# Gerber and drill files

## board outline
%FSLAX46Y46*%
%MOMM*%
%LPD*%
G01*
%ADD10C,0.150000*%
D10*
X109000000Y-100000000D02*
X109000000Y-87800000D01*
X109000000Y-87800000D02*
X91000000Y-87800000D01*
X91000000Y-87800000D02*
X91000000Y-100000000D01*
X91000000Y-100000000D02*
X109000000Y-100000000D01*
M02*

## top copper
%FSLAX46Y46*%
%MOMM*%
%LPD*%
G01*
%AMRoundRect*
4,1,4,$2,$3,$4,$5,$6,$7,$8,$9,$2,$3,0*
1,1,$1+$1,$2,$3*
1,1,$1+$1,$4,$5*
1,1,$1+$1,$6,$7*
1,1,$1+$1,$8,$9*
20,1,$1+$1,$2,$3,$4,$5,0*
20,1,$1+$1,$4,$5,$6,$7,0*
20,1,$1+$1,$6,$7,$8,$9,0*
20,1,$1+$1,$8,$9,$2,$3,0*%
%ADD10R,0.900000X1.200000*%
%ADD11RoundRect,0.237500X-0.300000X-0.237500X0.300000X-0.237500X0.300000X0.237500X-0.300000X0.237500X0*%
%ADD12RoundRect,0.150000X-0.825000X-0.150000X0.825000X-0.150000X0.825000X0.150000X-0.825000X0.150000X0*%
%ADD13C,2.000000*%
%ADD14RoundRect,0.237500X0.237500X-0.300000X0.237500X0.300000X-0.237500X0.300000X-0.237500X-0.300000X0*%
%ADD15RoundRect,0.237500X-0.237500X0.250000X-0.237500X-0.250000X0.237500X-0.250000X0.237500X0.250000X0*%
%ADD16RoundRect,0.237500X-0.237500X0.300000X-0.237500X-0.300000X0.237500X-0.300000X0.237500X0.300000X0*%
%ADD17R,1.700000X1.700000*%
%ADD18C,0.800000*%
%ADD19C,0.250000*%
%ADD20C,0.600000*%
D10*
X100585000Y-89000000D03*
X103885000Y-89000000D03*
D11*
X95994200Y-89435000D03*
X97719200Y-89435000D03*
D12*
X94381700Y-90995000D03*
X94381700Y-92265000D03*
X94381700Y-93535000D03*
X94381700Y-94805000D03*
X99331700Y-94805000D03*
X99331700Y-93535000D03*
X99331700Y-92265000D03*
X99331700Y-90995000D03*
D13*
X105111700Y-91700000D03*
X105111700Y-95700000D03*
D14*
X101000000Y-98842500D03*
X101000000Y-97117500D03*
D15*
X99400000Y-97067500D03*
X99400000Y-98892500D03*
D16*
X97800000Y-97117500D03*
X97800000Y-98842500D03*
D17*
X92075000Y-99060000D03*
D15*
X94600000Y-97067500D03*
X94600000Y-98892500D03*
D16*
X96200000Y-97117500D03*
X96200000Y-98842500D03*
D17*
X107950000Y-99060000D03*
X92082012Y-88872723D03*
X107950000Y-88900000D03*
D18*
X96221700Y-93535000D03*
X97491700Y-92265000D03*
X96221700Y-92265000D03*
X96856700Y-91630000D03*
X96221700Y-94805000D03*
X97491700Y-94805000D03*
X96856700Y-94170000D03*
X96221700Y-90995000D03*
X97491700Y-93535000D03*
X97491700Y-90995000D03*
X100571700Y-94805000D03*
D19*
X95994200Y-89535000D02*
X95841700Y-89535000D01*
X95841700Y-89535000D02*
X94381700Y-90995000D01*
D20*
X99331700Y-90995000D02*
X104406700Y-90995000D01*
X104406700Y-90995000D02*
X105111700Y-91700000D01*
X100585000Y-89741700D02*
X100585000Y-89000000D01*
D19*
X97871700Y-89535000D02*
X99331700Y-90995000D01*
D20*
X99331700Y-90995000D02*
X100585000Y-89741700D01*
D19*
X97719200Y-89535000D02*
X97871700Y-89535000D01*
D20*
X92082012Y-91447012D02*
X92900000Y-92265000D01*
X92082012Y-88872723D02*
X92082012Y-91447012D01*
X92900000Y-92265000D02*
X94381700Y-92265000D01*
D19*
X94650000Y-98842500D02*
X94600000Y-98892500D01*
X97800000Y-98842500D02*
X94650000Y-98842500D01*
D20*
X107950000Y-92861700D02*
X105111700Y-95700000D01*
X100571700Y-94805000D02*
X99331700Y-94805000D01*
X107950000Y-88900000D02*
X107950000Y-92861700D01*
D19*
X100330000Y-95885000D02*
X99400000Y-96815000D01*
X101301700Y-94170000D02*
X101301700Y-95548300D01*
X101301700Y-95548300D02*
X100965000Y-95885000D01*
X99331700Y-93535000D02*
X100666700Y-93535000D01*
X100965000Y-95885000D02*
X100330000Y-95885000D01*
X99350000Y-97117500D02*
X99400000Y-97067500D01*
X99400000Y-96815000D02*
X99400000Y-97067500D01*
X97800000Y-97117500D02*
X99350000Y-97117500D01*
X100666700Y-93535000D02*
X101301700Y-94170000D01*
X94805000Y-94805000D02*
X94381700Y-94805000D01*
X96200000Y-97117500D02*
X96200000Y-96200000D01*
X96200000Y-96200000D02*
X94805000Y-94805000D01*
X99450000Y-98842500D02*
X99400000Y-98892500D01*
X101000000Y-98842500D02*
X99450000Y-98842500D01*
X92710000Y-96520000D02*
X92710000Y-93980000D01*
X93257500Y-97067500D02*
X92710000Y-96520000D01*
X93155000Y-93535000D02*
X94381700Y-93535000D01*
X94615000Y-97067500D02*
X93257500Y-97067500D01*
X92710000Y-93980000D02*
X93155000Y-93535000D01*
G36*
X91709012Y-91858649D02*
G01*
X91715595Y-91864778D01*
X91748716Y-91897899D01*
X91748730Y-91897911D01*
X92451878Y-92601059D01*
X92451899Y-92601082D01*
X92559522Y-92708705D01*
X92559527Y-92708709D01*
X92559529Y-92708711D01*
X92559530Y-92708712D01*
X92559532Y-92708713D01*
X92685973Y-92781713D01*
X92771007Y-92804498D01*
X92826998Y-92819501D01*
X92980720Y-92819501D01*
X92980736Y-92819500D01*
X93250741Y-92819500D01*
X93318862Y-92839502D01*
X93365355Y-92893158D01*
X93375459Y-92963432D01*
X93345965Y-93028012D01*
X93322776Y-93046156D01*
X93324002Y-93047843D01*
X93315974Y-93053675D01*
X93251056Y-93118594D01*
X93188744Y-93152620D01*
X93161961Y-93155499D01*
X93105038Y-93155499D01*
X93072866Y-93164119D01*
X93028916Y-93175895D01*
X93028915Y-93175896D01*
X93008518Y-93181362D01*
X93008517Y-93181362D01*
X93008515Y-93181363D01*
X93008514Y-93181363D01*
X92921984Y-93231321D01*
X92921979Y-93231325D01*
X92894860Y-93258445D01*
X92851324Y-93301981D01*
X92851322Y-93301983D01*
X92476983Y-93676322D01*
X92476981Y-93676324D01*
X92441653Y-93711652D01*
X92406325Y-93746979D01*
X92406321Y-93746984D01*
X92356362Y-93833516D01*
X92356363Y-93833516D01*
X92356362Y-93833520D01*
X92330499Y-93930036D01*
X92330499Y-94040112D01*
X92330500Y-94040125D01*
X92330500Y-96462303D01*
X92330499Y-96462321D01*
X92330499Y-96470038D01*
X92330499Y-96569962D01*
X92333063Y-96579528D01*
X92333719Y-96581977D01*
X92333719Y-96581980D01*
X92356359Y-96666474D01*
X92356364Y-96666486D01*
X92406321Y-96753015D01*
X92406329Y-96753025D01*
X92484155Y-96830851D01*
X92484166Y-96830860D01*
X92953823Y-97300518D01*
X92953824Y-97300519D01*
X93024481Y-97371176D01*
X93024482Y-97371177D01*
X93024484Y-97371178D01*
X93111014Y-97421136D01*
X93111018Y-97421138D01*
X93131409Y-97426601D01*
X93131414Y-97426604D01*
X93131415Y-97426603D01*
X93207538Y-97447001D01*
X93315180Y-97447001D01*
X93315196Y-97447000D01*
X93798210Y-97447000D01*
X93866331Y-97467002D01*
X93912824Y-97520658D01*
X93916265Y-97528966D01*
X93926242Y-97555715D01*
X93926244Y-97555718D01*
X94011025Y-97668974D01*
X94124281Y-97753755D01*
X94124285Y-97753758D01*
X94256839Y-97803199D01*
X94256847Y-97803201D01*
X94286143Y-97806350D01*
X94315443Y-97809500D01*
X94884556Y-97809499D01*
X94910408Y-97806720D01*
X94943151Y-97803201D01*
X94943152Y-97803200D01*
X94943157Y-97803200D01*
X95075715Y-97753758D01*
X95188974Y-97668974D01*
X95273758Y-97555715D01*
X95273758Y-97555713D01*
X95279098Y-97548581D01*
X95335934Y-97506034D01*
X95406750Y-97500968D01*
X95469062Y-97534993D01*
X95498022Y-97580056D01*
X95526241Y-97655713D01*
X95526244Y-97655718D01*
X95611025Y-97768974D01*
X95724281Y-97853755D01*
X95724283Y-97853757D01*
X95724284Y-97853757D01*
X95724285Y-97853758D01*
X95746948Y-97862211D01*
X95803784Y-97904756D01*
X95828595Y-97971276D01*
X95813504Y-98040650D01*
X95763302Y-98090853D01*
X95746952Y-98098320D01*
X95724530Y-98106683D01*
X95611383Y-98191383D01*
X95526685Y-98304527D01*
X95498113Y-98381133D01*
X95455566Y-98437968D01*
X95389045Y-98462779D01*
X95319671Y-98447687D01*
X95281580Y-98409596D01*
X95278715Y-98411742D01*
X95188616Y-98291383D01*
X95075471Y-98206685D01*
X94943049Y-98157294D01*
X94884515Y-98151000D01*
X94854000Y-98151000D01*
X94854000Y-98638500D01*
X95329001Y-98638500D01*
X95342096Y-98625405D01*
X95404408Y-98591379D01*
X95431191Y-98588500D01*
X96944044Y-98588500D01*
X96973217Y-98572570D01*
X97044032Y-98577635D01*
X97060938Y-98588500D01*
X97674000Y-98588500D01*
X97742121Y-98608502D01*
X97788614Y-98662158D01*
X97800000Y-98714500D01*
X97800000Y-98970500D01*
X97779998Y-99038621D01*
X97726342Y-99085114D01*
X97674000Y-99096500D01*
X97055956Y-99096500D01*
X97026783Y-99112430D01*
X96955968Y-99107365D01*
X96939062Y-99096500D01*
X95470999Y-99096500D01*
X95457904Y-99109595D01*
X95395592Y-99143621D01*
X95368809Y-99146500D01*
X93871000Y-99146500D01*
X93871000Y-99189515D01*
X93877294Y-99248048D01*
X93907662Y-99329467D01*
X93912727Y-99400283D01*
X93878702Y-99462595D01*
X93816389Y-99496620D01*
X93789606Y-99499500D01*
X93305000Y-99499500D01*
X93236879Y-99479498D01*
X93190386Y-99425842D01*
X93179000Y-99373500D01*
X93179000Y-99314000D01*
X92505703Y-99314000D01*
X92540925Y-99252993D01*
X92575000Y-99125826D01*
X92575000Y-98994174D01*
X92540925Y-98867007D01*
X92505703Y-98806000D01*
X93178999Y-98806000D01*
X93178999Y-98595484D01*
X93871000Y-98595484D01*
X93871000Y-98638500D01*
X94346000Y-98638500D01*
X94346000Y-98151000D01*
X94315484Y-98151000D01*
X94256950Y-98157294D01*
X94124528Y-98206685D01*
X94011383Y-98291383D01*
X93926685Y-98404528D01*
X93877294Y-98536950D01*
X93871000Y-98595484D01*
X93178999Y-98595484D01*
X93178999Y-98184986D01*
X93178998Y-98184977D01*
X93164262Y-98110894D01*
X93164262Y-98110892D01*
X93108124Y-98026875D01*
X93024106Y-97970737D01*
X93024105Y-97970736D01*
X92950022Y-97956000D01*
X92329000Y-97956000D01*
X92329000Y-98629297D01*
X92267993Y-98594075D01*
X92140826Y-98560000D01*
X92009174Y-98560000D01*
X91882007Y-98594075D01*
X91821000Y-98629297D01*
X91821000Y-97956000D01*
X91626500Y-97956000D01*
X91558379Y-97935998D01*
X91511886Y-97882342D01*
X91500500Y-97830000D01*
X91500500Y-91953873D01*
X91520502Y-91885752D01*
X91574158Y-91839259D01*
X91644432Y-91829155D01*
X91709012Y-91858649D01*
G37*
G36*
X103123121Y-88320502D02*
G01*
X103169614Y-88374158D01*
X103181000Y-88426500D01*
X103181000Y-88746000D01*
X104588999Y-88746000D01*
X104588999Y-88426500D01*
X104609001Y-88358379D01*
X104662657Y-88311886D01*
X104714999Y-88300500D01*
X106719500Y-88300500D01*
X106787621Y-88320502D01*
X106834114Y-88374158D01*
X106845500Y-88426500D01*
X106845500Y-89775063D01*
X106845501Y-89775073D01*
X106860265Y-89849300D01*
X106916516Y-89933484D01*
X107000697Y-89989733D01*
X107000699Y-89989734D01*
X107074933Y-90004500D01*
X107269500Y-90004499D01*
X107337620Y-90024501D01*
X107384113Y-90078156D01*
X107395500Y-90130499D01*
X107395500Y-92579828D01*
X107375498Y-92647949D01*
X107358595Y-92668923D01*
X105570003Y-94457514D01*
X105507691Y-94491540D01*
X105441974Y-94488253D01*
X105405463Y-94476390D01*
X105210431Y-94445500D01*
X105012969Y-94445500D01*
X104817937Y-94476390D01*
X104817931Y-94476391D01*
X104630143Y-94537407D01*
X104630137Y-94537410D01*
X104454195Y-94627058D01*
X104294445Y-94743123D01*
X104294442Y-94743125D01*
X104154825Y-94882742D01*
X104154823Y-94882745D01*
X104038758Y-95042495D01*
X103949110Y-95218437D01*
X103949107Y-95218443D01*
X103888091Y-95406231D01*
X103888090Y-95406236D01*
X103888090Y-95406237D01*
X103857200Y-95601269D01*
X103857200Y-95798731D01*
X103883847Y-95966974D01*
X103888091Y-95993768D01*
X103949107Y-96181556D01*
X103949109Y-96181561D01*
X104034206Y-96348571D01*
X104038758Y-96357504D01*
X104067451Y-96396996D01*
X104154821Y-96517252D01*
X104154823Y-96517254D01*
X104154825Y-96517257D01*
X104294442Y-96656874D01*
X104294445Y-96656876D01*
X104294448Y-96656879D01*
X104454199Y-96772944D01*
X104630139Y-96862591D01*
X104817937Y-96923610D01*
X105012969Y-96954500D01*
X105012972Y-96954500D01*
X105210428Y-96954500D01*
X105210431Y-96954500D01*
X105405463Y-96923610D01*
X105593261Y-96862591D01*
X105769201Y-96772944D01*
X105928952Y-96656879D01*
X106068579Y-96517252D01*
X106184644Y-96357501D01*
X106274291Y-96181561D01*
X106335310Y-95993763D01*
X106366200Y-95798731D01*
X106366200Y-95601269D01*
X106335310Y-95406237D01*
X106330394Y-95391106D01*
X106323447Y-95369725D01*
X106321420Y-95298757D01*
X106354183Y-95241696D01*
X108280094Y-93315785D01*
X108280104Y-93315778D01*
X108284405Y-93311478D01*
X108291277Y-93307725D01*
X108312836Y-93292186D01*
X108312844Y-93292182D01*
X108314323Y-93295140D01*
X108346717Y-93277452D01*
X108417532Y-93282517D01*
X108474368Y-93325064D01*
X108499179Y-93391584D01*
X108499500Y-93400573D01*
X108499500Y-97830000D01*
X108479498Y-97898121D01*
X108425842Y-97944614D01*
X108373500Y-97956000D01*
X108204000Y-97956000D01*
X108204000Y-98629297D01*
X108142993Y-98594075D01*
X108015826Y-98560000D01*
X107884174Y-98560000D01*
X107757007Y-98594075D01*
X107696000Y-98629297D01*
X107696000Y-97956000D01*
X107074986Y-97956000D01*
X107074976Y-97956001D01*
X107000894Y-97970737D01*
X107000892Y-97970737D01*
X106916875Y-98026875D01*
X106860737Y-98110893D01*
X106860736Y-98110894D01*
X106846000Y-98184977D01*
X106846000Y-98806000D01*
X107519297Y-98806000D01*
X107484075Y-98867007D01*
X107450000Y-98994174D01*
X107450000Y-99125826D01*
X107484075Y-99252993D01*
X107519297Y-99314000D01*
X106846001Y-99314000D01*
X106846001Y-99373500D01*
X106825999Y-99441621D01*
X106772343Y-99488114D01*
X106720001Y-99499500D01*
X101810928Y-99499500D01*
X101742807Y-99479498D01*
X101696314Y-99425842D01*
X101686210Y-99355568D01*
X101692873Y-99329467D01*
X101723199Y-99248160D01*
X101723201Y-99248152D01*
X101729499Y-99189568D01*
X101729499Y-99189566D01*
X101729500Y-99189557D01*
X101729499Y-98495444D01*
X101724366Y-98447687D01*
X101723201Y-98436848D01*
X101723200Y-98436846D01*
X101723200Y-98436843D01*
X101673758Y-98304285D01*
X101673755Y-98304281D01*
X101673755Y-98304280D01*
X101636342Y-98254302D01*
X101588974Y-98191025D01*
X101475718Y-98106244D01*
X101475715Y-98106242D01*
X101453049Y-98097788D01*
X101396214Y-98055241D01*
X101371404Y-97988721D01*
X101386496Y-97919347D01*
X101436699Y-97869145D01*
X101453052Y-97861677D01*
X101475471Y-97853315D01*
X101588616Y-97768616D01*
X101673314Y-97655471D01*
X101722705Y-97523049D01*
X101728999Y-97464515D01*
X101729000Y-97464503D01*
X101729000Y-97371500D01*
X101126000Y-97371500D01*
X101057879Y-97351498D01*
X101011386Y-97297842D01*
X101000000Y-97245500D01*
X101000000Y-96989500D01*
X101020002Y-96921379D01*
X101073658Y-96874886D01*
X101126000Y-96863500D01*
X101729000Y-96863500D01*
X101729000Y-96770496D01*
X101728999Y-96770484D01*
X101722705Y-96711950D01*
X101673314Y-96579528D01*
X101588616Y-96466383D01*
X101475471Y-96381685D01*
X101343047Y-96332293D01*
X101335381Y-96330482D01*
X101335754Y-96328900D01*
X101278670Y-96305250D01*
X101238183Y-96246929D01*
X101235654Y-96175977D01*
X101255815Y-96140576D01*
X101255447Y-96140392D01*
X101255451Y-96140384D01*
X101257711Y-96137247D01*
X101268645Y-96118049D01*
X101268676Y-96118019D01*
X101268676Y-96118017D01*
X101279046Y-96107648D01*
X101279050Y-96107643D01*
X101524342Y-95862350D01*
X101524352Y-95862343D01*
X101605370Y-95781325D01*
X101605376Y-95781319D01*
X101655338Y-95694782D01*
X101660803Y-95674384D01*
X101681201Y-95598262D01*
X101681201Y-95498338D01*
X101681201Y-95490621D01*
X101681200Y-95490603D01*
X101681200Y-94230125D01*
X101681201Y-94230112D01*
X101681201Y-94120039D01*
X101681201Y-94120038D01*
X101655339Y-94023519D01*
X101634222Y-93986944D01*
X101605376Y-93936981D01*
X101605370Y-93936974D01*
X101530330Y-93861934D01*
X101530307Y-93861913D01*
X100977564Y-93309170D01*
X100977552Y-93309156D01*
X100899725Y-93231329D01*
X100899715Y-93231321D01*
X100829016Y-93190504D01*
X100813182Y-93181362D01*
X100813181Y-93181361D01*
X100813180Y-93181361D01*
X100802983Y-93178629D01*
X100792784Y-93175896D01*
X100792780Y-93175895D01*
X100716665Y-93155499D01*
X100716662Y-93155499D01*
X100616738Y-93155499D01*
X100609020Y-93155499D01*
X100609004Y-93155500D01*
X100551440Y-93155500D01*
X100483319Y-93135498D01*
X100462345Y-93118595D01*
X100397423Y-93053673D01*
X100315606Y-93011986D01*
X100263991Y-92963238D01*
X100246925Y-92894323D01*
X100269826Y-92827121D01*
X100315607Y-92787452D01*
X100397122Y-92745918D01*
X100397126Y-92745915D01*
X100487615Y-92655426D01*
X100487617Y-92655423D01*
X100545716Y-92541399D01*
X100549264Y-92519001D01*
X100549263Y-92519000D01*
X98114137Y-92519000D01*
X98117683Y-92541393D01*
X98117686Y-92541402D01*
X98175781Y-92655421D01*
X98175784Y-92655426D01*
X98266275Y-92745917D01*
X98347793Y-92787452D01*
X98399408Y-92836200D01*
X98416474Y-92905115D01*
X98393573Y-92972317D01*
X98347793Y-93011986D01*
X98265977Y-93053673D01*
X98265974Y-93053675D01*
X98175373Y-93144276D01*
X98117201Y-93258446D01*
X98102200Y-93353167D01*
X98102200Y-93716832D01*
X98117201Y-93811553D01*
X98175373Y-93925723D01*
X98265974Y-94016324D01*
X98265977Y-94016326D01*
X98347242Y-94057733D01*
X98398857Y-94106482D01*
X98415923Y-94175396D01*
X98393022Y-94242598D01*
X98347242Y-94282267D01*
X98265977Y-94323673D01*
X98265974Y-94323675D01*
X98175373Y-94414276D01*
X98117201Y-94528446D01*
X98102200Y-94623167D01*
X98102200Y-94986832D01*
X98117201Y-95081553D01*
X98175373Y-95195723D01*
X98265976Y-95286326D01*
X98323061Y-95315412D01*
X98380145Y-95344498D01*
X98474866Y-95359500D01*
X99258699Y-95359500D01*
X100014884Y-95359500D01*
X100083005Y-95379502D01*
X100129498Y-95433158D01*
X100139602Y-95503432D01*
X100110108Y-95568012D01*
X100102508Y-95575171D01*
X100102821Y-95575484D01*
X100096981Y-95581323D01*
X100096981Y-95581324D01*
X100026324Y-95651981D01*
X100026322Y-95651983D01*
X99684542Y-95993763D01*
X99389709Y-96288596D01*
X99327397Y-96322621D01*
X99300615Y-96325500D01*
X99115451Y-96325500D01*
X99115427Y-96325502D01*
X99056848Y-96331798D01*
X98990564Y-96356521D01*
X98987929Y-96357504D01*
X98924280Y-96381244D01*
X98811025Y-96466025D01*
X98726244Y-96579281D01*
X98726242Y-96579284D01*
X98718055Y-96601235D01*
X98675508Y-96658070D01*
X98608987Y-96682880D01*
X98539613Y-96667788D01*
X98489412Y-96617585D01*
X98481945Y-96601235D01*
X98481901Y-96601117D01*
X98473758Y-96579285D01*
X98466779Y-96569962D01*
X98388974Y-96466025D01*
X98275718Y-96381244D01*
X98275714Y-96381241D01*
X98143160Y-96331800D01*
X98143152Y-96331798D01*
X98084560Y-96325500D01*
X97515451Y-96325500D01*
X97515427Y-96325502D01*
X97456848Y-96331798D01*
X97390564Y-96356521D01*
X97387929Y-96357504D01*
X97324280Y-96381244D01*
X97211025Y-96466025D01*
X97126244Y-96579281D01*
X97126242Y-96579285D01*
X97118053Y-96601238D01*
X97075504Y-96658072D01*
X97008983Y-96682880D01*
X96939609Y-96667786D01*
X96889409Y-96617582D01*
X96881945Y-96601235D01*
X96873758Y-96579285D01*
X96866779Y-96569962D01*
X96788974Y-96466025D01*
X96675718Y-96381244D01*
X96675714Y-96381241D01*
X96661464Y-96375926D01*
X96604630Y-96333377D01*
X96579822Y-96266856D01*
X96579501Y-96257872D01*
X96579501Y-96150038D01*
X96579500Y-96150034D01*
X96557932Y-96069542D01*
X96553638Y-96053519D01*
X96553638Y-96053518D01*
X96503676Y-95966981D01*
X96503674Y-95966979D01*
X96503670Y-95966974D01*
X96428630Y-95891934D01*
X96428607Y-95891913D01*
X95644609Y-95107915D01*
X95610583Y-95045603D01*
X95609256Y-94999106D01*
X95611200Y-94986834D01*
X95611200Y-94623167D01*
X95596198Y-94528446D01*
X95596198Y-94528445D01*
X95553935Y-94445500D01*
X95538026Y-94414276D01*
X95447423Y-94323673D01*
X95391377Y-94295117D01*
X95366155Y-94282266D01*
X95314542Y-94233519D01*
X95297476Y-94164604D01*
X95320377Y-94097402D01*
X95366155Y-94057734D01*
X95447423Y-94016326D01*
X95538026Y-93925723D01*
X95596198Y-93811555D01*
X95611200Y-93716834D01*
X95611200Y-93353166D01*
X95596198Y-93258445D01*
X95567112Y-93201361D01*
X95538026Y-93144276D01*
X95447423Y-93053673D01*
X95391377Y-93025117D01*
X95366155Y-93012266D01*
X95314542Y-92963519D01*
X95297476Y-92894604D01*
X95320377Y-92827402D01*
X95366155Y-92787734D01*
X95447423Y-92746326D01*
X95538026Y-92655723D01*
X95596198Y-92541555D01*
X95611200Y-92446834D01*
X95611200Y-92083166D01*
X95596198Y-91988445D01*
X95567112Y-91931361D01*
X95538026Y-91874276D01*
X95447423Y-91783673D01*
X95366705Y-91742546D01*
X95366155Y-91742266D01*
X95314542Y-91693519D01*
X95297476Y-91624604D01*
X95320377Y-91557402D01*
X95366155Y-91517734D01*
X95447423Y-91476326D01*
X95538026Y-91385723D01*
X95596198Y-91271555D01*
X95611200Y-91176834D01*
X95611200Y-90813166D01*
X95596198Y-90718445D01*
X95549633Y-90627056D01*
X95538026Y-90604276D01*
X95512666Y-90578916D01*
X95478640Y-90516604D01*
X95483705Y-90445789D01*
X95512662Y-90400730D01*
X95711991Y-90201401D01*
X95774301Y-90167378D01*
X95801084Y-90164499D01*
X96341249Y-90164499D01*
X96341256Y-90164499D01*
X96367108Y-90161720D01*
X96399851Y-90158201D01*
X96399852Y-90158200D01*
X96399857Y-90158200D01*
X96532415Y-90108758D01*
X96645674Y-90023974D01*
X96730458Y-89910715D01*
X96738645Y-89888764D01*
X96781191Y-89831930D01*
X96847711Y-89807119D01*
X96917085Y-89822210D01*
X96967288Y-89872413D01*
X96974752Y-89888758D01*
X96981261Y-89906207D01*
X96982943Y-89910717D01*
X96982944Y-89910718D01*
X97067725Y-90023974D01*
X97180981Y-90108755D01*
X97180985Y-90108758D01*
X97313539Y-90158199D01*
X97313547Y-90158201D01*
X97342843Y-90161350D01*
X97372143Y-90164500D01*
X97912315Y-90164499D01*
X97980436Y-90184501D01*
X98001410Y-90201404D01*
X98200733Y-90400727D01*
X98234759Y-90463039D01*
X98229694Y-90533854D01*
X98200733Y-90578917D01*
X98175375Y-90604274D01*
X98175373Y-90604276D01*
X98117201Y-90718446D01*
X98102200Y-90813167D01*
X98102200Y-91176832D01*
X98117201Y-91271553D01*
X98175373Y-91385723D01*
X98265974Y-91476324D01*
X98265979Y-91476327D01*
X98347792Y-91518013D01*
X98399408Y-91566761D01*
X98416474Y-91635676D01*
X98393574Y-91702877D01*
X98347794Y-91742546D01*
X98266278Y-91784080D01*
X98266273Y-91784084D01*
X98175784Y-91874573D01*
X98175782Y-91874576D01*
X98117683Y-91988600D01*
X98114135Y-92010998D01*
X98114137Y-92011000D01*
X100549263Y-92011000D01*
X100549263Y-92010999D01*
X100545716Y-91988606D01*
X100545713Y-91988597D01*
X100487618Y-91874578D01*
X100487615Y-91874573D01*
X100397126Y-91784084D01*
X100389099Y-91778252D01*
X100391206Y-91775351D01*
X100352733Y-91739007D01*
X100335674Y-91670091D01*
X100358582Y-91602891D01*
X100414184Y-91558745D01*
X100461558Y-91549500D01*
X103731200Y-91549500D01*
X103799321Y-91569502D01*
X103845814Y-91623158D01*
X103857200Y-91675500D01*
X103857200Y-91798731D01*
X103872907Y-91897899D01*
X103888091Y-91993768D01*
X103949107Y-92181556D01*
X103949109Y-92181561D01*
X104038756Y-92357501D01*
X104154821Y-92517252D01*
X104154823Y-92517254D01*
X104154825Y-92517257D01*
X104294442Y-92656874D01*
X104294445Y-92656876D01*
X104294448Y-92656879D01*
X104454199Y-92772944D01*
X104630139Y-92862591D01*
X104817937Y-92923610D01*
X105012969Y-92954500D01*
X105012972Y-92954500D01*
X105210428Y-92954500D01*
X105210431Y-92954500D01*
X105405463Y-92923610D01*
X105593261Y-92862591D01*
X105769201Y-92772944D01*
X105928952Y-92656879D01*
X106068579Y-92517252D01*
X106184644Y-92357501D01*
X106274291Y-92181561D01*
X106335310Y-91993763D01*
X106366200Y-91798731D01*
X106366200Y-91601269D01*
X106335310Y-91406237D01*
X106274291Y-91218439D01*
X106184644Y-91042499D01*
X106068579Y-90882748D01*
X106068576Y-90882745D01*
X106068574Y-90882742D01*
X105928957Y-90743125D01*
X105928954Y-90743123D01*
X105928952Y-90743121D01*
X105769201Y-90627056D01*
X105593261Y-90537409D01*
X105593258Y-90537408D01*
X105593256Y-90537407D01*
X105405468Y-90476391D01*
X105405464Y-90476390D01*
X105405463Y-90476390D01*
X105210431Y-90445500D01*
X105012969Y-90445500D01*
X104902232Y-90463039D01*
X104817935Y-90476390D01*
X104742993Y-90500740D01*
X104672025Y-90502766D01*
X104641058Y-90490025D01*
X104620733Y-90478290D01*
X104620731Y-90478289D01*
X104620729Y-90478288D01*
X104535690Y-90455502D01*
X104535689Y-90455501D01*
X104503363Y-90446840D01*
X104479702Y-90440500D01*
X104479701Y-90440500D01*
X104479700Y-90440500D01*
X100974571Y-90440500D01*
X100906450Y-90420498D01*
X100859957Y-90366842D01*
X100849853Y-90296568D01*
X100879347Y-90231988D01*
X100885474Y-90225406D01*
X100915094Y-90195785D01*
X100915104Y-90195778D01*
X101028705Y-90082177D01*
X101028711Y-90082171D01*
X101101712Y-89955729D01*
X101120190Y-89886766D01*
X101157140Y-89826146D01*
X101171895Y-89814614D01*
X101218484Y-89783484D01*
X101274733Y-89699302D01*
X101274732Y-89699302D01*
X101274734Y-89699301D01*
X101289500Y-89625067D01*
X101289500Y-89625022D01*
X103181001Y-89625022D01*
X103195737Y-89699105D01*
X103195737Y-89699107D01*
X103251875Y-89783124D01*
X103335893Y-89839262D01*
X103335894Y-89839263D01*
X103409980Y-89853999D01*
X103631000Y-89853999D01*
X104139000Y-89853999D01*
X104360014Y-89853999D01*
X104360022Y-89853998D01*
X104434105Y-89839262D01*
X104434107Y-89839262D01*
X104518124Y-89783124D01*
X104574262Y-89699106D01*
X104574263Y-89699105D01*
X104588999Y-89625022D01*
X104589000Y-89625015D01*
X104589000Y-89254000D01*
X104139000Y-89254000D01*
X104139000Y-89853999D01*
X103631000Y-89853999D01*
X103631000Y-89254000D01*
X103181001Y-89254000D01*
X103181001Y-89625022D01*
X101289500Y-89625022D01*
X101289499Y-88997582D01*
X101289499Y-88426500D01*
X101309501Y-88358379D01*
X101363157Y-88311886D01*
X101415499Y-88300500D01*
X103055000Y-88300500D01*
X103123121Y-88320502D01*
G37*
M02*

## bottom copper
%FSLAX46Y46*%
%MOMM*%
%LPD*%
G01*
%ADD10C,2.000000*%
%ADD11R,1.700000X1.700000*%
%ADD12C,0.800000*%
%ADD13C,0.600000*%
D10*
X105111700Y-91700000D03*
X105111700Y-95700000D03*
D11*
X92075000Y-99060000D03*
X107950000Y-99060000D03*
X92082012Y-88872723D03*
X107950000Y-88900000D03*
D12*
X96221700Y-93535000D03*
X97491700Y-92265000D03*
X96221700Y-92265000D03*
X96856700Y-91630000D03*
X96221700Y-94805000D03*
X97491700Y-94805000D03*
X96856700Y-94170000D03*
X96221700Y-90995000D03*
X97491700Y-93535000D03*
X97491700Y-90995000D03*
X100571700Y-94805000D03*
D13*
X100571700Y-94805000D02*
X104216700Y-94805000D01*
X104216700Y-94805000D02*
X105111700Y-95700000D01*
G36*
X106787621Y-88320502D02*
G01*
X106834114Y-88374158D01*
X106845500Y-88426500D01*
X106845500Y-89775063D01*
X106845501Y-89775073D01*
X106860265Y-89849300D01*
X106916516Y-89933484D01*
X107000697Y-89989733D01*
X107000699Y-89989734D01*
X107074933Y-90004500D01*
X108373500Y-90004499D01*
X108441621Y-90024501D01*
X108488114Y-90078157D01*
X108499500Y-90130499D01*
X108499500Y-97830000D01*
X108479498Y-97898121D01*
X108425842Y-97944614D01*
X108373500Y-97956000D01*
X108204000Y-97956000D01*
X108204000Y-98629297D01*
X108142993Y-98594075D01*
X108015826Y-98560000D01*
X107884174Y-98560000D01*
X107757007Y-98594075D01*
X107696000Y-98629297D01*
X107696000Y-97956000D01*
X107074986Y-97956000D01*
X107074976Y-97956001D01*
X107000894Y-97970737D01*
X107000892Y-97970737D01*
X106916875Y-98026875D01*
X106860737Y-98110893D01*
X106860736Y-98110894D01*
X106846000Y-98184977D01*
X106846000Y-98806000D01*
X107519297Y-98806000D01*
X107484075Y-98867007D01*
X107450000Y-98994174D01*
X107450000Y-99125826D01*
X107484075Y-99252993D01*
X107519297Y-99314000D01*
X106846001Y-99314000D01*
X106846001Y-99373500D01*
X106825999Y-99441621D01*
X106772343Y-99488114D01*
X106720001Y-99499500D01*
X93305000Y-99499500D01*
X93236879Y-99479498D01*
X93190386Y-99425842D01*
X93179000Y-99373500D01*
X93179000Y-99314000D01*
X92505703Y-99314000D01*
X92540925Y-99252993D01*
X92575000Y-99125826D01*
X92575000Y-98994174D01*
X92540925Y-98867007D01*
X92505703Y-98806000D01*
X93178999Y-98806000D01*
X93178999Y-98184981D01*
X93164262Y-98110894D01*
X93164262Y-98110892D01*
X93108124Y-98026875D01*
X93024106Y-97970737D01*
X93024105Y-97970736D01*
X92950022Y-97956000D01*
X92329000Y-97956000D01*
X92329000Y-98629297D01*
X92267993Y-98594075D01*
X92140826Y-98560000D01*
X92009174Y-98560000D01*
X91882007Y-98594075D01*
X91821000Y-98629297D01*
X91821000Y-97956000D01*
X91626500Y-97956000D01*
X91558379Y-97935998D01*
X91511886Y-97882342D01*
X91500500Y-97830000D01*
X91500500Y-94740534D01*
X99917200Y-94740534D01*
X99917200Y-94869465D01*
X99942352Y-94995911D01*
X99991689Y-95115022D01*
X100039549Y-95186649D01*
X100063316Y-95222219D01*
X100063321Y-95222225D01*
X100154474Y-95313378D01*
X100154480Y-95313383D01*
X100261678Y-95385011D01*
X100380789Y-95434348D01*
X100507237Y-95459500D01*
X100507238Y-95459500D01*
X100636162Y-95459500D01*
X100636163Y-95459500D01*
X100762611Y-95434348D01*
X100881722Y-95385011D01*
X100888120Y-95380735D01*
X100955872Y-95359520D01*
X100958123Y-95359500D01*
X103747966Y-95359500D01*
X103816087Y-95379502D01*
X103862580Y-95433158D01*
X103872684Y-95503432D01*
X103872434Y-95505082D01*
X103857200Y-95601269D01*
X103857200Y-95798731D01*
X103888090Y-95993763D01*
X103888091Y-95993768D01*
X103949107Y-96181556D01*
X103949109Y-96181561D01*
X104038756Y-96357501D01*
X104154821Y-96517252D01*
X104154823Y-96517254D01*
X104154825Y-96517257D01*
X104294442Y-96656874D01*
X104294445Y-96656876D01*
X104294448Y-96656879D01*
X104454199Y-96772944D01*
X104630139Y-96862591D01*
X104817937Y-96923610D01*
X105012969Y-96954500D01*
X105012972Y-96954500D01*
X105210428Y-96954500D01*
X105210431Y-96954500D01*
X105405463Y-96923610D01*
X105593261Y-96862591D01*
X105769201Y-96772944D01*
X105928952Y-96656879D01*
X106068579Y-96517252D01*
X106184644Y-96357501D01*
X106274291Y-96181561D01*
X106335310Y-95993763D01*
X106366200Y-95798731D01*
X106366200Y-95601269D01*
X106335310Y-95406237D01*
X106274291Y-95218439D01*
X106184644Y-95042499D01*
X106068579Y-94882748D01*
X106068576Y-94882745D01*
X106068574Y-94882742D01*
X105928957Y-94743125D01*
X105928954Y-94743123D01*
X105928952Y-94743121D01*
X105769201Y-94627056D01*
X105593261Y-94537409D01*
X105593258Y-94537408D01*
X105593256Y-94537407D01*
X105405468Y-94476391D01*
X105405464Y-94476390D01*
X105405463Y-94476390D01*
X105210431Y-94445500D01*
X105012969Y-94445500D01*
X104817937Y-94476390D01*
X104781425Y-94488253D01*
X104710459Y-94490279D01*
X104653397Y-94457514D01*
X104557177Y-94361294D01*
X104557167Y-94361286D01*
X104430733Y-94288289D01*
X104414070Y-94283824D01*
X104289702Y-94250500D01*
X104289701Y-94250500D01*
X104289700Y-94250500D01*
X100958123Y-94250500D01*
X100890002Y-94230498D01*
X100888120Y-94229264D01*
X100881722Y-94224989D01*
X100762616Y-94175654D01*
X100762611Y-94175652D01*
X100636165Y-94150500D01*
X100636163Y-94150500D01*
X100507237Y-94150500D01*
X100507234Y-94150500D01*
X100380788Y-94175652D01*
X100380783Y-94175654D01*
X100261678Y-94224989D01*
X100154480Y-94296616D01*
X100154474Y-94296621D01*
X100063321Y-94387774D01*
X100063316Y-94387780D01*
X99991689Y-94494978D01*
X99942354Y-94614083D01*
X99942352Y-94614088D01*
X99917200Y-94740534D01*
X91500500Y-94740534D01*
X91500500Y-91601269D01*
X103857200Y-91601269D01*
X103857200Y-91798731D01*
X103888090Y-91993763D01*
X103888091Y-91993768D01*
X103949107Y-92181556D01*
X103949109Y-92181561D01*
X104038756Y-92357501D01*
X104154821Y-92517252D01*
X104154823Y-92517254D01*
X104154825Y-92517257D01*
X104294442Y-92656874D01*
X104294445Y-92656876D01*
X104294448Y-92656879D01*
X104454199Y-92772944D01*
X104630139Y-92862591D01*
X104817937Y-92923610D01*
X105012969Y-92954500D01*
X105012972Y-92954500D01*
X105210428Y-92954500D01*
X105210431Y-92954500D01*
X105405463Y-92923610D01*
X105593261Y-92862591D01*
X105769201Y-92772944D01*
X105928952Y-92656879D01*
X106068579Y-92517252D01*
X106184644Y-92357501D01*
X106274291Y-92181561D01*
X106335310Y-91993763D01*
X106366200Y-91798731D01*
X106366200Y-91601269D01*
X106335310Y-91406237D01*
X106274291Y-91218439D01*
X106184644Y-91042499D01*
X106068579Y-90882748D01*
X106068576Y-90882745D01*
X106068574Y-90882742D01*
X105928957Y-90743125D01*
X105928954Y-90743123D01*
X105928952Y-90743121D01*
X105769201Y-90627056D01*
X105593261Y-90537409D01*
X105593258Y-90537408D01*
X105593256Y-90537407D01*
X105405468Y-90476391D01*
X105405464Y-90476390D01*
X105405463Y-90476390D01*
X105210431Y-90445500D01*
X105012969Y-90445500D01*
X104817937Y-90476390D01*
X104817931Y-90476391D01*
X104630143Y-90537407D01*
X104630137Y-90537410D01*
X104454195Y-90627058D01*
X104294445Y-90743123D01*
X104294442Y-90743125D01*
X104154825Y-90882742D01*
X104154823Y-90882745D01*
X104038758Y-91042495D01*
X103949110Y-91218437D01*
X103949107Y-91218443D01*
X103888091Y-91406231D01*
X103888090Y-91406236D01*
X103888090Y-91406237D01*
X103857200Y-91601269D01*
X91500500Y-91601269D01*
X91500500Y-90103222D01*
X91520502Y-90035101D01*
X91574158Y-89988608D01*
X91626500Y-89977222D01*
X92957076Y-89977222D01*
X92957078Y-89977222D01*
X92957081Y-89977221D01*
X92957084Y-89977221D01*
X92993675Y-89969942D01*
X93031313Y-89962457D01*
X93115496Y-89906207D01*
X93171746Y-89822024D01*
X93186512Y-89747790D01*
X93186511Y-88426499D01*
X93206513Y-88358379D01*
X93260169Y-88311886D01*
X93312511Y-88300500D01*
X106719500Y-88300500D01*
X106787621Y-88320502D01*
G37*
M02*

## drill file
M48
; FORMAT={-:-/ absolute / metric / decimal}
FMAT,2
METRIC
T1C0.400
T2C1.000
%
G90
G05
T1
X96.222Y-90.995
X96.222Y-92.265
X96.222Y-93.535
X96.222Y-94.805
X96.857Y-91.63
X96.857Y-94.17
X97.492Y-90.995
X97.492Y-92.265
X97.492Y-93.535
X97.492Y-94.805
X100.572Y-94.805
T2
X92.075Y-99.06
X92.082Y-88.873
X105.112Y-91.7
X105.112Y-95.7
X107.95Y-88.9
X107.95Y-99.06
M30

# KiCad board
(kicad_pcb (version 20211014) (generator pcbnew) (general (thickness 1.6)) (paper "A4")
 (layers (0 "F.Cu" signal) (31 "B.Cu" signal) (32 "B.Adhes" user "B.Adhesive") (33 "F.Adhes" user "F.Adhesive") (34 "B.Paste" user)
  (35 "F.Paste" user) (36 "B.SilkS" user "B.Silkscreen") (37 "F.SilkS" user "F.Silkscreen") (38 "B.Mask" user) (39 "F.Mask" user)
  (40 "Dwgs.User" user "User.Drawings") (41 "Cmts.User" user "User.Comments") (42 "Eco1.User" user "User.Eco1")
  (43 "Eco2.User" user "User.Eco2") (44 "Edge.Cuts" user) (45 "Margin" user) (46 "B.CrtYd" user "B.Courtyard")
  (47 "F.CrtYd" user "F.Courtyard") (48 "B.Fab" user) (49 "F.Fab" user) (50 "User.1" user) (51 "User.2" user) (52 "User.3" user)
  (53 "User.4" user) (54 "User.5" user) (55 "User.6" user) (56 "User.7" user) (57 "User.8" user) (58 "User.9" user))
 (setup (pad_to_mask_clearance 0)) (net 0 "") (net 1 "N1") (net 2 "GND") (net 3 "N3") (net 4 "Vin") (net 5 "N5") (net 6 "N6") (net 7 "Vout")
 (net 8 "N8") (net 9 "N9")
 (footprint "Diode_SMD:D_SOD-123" (layer "F.Cu") (at 102.235 89)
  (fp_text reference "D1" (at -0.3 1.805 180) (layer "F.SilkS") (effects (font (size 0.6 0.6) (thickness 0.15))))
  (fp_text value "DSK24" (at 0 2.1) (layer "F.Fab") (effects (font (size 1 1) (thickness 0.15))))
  (pad "1" smd rect (at -1.65 0) (size 0.9 1.2) (layers "F.Cu" "F.Paste" "F.Mask") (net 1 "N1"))
  (pad "2" smd rect (at 1.65 0) (size 0.9 1.2) (layers "F.Cu" "F.Paste" "F.Mask") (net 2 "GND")))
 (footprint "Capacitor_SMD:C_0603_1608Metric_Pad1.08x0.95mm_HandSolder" (layer "F.Cu") (at 96.8567 89.435)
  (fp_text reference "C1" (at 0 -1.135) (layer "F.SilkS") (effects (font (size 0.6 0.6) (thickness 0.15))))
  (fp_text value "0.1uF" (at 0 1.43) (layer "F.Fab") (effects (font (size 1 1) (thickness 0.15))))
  (pad "1" smd roundrect (at -0.8625 0) (size 1.075 0.95) (layers "F.Cu" "F.Paste" "F.Mask") (roundrect_rratio 0.25) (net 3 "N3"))
  (pad "2" smd roundrect (at 0.8625 0) (size 1.075 0.95) (layers "F.Cu" "F.Paste" "F.Mask") (roundrect_rratio 0.25) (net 1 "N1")))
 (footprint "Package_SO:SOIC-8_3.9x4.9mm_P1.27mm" (layer "F.Cu") (at 96.8567 92.9)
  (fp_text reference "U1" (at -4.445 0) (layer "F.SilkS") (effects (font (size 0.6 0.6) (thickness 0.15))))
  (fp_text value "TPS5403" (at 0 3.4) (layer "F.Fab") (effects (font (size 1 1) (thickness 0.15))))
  (pad "1" smd roundrect (at -2.475 -1.905) (size 1.95 0.6) (layers "F.Cu" "F.Paste" "F.Mask") (roundrect_rratio 0.25) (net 3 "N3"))
  (pad "2" smd roundrect (at -2.475 -0.635) (size 1.95 0.6) (layers "F.Cu" "F.Paste" "F.Mask") (roundrect_rratio 0.25) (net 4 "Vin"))
  (pad "3" smd roundrect (at -2.475 0.635) (size 1.95 0.6) (layers "F.Cu" "F.Paste" "F.Mask") (roundrect_rratio 0.25) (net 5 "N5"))
  (pad "4" smd roundrect (at -2.475 1.905) (size 1.95 0.6) (layers "F.Cu" "F.Paste" "F.Mask") (roundrect_rratio 0.25) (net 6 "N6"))
  (pad "5" smd roundrect (at 2.475 1.905) (size 1.95 0.6) (layers "F.Cu" "F.Paste" "F.Mask") (roundrect_rratio 0.25) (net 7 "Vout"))
  (pad "6" smd roundrect (at 2.475 0.635) (size 1.95 0.6) (layers "F.Cu" "F.Paste" "F.Mask") (roundrect_rratio 0.25) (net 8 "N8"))
  (pad "7" smd roundrect (at 2.475 -0.635) (size 1.95 0.6) (layers "F.Cu" "F.Paste" "F.Mask") (roundrect_rratio 0.25) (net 2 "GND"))
  (pad "8" smd roundrect (at 2.475 -1.905) (size 1.95 0.6) (layers "F.Cu" "F.Paste" "F.Mask") (roundrect_rratio 0.25) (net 1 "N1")))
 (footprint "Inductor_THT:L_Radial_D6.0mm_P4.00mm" (layer "F.Cu") (at 105.1117 91.7 -90)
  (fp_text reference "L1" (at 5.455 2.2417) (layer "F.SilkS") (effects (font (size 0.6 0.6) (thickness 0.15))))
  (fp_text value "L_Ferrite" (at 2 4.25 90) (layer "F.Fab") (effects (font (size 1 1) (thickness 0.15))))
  (pad "1" thru_hole circle (at 0 0 270) (size 2 2) (drill 1) (layers *.Cu *.Mask) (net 1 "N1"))
  (pad "2" thru_hole circle (at 4 0 270) (size 2 2) (drill 1) (layers *.Cu *.Mask) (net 7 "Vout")))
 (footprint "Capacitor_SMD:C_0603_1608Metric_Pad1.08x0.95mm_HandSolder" (layer "F.Cu") (at 101 97.98 90)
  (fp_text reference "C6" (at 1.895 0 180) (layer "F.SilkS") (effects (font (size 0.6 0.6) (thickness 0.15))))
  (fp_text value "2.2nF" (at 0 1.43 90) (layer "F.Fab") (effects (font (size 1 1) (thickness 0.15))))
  (pad "1" smd roundrect (at -0.8625 0 90) (size 1.075 0.95) (layers "F.Cu" "F.Paste" "F.Mask") (roundrect_rratio 0.25) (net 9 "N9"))
  (pad "2" smd roundrect (at 0.8625 0 90) (size 1.075 0.95) (layers "F.Cu" "F.Paste" "F.Mask") (roundrect_rratio 0.25) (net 2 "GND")))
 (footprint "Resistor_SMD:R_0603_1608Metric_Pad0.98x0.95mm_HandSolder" (layer "F.Cu") (at 99.4 97.98 -90)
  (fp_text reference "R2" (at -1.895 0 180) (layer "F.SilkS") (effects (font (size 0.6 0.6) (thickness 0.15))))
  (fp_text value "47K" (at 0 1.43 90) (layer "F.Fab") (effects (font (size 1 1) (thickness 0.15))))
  (pad "1" smd roundrect (at -0.9125 0 270) (size 0.975 0.95) (layers "F.Cu" "F.Paste" "F.Mask") (roundrect_rratio 0.25) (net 8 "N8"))
  (pad "2" smd roundrect (at 0.9125 0 270) (size 0.975 0.95) (layers "F.Cu" "F.Paste" "F.Mask") (roundrect_rratio 0.25) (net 9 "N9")))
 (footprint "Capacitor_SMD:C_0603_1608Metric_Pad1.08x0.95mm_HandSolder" (layer "F.Cu") (at 97.8 97.98 -90)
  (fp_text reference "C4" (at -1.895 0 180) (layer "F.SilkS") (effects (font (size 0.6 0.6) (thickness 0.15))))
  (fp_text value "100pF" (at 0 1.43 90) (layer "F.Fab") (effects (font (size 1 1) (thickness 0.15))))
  (pad "1" smd roundrect (at -0.8625 0 270) (size 1.075 0.95) (layers "F.Cu" "F.Paste" "F.Mask") (roundrect_rratio 0.25) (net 8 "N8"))
  (pad "2" smd roundrect (at 0.8625 0 270) (size 1.075 0.95) (layers "F.Cu" "F.Paste" "F.Mask") (roundrect_rratio 0.25) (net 2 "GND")))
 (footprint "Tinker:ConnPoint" (layer "F.Cu") (at 92.075 99.06)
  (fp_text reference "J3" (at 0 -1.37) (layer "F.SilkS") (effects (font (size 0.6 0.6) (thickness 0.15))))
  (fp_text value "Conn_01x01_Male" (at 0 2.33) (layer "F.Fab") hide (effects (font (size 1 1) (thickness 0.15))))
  (pad "1" thru_hole rect (at 0 0) (size 1.7 1.7) (drill 1) (layers *.Cu *.Mask) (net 2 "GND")))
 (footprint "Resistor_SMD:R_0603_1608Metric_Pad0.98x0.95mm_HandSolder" (layer "F.Cu") (at 94.6 97.98 -90)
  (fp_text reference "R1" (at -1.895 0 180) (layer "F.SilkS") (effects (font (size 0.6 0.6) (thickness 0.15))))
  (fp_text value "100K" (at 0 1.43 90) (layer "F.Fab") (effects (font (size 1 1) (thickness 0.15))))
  (pad "1" smd roundrect (at -0.9125 0 270) (size 0.975 0.95) (layers "F.Cu" "F.Paste" "F.Mask") (roundrect_rratio 0.25) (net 5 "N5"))
  (pad "2" smd roundrect (at 0.9125 0 270) (size 0.975 0.95) (layers "F.Cu" "F.Paste" "F.Mask") (roundrect_rratio 0.25) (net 2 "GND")))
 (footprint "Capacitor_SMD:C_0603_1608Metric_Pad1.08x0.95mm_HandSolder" (layer "F.Cu") (at 96.2 97.98 -90)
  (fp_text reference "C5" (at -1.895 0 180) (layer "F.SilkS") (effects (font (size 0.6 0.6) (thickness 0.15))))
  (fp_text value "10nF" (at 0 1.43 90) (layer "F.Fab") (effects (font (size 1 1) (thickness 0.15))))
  (pad "1" smd roundrect (at -0.8625 0 270) (size 1.075 0.95) (layers "F.Cu" "F.Paste" "F.Mask") (roundrect_rratio 0.25) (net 6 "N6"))
  (pad "2" smd roundrect (at 0.8625 0 270) (size 1.075 0.95) (layers "F.Cu" "F.Paste" "F.Mask") (roundrect_rratio 0.25) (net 2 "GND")))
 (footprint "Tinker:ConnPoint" (layer "F.Cu") (at 107.95 99.06)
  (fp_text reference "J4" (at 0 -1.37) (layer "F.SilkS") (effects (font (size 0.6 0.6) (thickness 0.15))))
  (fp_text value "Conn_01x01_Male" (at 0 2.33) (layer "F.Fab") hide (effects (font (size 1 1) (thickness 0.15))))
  (pad "1" thru_hole rect (at 0 0) (size 1.7 1.7) (drill 1) (layers *.Cu *.Mask) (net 2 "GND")))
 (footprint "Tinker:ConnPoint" (layer "F.Cu") (at 92.082012 88.872723)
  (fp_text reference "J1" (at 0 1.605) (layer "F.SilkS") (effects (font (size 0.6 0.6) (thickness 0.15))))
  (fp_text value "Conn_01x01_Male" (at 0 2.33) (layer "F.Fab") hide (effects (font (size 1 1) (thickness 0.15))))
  (pad "1" thru_hole rect (at 0 0) (size 1.7 1.7) (drill 1) (layers *.Cu *.Mask) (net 4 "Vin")))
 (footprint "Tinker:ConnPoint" (layer "F.Cu") (at 107.95 88.9)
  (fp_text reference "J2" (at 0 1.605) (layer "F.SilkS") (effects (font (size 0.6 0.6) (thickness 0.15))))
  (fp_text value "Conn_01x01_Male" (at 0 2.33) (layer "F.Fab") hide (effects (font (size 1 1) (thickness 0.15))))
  (pad "1" thru_hole rect (at 0 0) (size 1.7 1.7) (drill 1) (layers *.Cu *.Mask) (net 7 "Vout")))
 (gr_line (start 109 100) (end 109 87.8) (layer "Edge.Cuts") (width 0.15))
 (gr_line (start 109 87.8) (end 91 87.8) (layer "Edge.Cuts") (width 0.15))
 (gr_line (start 91 87.8) (end 91 100) (layer "Edge.Cuts") (width 0.15))
 (gr_line (start 91 100) (end 109 100) (layer "Edge.Cuts") (width 0.15))
 (segment (start 95.9942 89.535) (end 95.8417 89.535) (width 0.25) (layer "F.Cu") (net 3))
 (segment (start 95.8417 89.535) (end 94.3817 90.995) (width 0.25) (layer "F.Cu") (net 3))
 (segment (start 99.3317 90.995) (end 104.4067 90.995) (width 0.6) (layer "F.Cu") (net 1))
 (segment (start 104.4067 90.995) (end 105.1117 91.7) (width 0.6) (layer "F.Cu") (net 1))
 (segment (start 100.585 89.7417) (end 100.585 89) (width 0.6) (layer "F.Cu") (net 1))
 (segment (start 97.8717 89.535) (end 99.3317 90.995) (width 0.25) (layer "F.Cu") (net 1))
 (segment (start 99.3317 90.995) (end 100.585 89.7417) (width 0.6) (layer "F.Cu") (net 1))
 (segment (start 97.7192 89.535) (end 97.8717 89.535) (width 0.25) (layer "F.Cu") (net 1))
 (segment (start 92.082012 91.447012) (end 92.9 92.265) (width 0.6) (layer "F.Cu") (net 4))
 (segment (start 92.082012 88.872723) (end 92.082012 91.447012) (width 0.6) (layer "F.Cu") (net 4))
 (segment (start 92.9 92.265) (end 94.3817 92.265) (width 0.6) (layer "F.Cu") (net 4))
 (segment (start 94.65 98.8425) (end 94.6 98.8925) (width 0.25) (layer "F.Cu") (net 2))
 (segment (start 97.8 98.8425) (end 94.65 98.8425) (width 0.25) (layer "F.Cu") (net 2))
 (via (at 96.2217 93.535) (size 0.8) (drill 0.4) (layers "F.Cu" "B.Cu") (free) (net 2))
 (via (at 97.4917 92.265) (size 0.8) (drill 0.4) (layers "F.Cu" "B.Cu") (free) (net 2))
 (via (at 96.2217 92.265) (size 0.8) (drill 0.4) (layers "F.Cu" "B.Cu") (free) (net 2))
 (via (at 96.8567 91.63) (size 0.8) (drill 0.4) (layers "F.Cu" "B.Cu") (free) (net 2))
 (via (at 96.2217 94.805) (size 0.8) (drill 0.4) (layers "F.Cu" "B.Cu") (free) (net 2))
 (via (at 97.4917 94.805) (size 0.8) (drill 0.4) (layers "F.Cu" "B.Cu") (free) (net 2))
 (via (at 96.8567 94.17) (size 0.8) (drill 0.4) (layers "F.Cu" "B.Cu") (free) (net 2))
 (via (at 96.2217 90.995) (size 0.8) (drill 0.4) (layers "F.Cu" "B.Cu") (free) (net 2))
 (via (at 97.4917 93.535) (size 0.8) (drill 0.4) (layers "F.Cu" "B.Cu") (free) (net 2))
 (via (at 97.4917 90.995) (size 0.8) (drill 0.4) (layers "F.Cu" "B.Cu") (free) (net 2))
 (segment (start 107.95 92.8617) (end 105.1117 95.7) (width 0.6) (layer "F.Cu") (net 7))
 (segment (start 100.5717 94.805) (end 99.3317 94.805) (width 0.6) (layer "F.Cu") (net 7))
 (segment (start 107.95 88.9) (end 107.95 92.8617) (width 0.6) (layer "F.Cu") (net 7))
 (via (at 100.5717 94.805) (size 0.8) (drill 0.4) (layers "F.Cu" "B.Cu") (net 7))
 (segment (start 100.5717 94.805) (end 104.2167 94.805) (width 0.6) (layer "B.Cu") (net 7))
 (segment (start 104.2167 94.805) (end 105.1117 95.7) (width 0.6) (layer "B.Cu") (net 7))
 (segment (start 100.33 95.885) (end 99.4 96.815) (width 0.25) (layer "F.Cu") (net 8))
 (segment (start 101.3017 94.17) (end 101.3017 95.5483) (width 0.25) (layer "F.Cu") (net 8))
 (segment (start 101.3017 95.5483) (end 100.965 95.885) (width 0.25) (layer "F.Cu") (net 8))
 (segment (start 99.3317 93.535) (end 100.6667 93.535) (width 0.25) (layer "F.Cu") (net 8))
 (segment (start 100.965 95.885) (end 100.33 95.885) (width 0.25) (layer "F.Cu") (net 8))
 (segment (start 99.35 97.1175) (end 99.4 97.0675) (width 0.25) (layer "F.Cu") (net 8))
 (segment (start 99.4 96.815) (end 99.4 97.0675) (width 0.25) (layer "F.Cu") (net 8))
 (segment (start 97.8 97.1175) (end 99.35 97.1175) (width 0.25) (layer "F.Cu") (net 8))
 (segment (start 100.6667 93.535) (end 101.3017 94.17) (width 0.25) (layer "F.Cu") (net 8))
 (segment (start 94.805 94.805) (end 94.3817 94.805) (width 0.25) (layer "F.Cu") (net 6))
 (segment (start 96.2 97.1175) (end 96.2 96.2) (width 0.25) (layer "F.Cu") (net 6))
 (segment (start 96.2 96.2) (end 94.805 94.805) (width 0.25) (layer "F.Cu") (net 6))
 (segment (start 99.45 98.8425) (end 99.4 98.8925) (width 0.25) (layer "F.Cu") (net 9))
 (segment (start 101 98.8425) (end 99.45 98.8425) (width 0.25) (layer "F.Cu") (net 9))
 (segment (start 92.71 96.52) (end 92.71 93.98) (width 0.25) (layer "F.Cu") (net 5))
 (segment (start 93.2575 97.0675) (end 92.71 96.52) (width 0.25) (layer "F.Cu") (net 5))
 (segment (start 93.155 93.535) (end 94.3817 93.535) (width 0.25) (layer "F.Cu") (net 5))
 (segment (start 94.615 97.0675) (end 93.2575 97.0675) (width 0.25) (layer "F.Cu") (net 5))
 (segment (start 92.71 93.98) (end 93.155 93.535) (width 0.25) (layer "F.Cu") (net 5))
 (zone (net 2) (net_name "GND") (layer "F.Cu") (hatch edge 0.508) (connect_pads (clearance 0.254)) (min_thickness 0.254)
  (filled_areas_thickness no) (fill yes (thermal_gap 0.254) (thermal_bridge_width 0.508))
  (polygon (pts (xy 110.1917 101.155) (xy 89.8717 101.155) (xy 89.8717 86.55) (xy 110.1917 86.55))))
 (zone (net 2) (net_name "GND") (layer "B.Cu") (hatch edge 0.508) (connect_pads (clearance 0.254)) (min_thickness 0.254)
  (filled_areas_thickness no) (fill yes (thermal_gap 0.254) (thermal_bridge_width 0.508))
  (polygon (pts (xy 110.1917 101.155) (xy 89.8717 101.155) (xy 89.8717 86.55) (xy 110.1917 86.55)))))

